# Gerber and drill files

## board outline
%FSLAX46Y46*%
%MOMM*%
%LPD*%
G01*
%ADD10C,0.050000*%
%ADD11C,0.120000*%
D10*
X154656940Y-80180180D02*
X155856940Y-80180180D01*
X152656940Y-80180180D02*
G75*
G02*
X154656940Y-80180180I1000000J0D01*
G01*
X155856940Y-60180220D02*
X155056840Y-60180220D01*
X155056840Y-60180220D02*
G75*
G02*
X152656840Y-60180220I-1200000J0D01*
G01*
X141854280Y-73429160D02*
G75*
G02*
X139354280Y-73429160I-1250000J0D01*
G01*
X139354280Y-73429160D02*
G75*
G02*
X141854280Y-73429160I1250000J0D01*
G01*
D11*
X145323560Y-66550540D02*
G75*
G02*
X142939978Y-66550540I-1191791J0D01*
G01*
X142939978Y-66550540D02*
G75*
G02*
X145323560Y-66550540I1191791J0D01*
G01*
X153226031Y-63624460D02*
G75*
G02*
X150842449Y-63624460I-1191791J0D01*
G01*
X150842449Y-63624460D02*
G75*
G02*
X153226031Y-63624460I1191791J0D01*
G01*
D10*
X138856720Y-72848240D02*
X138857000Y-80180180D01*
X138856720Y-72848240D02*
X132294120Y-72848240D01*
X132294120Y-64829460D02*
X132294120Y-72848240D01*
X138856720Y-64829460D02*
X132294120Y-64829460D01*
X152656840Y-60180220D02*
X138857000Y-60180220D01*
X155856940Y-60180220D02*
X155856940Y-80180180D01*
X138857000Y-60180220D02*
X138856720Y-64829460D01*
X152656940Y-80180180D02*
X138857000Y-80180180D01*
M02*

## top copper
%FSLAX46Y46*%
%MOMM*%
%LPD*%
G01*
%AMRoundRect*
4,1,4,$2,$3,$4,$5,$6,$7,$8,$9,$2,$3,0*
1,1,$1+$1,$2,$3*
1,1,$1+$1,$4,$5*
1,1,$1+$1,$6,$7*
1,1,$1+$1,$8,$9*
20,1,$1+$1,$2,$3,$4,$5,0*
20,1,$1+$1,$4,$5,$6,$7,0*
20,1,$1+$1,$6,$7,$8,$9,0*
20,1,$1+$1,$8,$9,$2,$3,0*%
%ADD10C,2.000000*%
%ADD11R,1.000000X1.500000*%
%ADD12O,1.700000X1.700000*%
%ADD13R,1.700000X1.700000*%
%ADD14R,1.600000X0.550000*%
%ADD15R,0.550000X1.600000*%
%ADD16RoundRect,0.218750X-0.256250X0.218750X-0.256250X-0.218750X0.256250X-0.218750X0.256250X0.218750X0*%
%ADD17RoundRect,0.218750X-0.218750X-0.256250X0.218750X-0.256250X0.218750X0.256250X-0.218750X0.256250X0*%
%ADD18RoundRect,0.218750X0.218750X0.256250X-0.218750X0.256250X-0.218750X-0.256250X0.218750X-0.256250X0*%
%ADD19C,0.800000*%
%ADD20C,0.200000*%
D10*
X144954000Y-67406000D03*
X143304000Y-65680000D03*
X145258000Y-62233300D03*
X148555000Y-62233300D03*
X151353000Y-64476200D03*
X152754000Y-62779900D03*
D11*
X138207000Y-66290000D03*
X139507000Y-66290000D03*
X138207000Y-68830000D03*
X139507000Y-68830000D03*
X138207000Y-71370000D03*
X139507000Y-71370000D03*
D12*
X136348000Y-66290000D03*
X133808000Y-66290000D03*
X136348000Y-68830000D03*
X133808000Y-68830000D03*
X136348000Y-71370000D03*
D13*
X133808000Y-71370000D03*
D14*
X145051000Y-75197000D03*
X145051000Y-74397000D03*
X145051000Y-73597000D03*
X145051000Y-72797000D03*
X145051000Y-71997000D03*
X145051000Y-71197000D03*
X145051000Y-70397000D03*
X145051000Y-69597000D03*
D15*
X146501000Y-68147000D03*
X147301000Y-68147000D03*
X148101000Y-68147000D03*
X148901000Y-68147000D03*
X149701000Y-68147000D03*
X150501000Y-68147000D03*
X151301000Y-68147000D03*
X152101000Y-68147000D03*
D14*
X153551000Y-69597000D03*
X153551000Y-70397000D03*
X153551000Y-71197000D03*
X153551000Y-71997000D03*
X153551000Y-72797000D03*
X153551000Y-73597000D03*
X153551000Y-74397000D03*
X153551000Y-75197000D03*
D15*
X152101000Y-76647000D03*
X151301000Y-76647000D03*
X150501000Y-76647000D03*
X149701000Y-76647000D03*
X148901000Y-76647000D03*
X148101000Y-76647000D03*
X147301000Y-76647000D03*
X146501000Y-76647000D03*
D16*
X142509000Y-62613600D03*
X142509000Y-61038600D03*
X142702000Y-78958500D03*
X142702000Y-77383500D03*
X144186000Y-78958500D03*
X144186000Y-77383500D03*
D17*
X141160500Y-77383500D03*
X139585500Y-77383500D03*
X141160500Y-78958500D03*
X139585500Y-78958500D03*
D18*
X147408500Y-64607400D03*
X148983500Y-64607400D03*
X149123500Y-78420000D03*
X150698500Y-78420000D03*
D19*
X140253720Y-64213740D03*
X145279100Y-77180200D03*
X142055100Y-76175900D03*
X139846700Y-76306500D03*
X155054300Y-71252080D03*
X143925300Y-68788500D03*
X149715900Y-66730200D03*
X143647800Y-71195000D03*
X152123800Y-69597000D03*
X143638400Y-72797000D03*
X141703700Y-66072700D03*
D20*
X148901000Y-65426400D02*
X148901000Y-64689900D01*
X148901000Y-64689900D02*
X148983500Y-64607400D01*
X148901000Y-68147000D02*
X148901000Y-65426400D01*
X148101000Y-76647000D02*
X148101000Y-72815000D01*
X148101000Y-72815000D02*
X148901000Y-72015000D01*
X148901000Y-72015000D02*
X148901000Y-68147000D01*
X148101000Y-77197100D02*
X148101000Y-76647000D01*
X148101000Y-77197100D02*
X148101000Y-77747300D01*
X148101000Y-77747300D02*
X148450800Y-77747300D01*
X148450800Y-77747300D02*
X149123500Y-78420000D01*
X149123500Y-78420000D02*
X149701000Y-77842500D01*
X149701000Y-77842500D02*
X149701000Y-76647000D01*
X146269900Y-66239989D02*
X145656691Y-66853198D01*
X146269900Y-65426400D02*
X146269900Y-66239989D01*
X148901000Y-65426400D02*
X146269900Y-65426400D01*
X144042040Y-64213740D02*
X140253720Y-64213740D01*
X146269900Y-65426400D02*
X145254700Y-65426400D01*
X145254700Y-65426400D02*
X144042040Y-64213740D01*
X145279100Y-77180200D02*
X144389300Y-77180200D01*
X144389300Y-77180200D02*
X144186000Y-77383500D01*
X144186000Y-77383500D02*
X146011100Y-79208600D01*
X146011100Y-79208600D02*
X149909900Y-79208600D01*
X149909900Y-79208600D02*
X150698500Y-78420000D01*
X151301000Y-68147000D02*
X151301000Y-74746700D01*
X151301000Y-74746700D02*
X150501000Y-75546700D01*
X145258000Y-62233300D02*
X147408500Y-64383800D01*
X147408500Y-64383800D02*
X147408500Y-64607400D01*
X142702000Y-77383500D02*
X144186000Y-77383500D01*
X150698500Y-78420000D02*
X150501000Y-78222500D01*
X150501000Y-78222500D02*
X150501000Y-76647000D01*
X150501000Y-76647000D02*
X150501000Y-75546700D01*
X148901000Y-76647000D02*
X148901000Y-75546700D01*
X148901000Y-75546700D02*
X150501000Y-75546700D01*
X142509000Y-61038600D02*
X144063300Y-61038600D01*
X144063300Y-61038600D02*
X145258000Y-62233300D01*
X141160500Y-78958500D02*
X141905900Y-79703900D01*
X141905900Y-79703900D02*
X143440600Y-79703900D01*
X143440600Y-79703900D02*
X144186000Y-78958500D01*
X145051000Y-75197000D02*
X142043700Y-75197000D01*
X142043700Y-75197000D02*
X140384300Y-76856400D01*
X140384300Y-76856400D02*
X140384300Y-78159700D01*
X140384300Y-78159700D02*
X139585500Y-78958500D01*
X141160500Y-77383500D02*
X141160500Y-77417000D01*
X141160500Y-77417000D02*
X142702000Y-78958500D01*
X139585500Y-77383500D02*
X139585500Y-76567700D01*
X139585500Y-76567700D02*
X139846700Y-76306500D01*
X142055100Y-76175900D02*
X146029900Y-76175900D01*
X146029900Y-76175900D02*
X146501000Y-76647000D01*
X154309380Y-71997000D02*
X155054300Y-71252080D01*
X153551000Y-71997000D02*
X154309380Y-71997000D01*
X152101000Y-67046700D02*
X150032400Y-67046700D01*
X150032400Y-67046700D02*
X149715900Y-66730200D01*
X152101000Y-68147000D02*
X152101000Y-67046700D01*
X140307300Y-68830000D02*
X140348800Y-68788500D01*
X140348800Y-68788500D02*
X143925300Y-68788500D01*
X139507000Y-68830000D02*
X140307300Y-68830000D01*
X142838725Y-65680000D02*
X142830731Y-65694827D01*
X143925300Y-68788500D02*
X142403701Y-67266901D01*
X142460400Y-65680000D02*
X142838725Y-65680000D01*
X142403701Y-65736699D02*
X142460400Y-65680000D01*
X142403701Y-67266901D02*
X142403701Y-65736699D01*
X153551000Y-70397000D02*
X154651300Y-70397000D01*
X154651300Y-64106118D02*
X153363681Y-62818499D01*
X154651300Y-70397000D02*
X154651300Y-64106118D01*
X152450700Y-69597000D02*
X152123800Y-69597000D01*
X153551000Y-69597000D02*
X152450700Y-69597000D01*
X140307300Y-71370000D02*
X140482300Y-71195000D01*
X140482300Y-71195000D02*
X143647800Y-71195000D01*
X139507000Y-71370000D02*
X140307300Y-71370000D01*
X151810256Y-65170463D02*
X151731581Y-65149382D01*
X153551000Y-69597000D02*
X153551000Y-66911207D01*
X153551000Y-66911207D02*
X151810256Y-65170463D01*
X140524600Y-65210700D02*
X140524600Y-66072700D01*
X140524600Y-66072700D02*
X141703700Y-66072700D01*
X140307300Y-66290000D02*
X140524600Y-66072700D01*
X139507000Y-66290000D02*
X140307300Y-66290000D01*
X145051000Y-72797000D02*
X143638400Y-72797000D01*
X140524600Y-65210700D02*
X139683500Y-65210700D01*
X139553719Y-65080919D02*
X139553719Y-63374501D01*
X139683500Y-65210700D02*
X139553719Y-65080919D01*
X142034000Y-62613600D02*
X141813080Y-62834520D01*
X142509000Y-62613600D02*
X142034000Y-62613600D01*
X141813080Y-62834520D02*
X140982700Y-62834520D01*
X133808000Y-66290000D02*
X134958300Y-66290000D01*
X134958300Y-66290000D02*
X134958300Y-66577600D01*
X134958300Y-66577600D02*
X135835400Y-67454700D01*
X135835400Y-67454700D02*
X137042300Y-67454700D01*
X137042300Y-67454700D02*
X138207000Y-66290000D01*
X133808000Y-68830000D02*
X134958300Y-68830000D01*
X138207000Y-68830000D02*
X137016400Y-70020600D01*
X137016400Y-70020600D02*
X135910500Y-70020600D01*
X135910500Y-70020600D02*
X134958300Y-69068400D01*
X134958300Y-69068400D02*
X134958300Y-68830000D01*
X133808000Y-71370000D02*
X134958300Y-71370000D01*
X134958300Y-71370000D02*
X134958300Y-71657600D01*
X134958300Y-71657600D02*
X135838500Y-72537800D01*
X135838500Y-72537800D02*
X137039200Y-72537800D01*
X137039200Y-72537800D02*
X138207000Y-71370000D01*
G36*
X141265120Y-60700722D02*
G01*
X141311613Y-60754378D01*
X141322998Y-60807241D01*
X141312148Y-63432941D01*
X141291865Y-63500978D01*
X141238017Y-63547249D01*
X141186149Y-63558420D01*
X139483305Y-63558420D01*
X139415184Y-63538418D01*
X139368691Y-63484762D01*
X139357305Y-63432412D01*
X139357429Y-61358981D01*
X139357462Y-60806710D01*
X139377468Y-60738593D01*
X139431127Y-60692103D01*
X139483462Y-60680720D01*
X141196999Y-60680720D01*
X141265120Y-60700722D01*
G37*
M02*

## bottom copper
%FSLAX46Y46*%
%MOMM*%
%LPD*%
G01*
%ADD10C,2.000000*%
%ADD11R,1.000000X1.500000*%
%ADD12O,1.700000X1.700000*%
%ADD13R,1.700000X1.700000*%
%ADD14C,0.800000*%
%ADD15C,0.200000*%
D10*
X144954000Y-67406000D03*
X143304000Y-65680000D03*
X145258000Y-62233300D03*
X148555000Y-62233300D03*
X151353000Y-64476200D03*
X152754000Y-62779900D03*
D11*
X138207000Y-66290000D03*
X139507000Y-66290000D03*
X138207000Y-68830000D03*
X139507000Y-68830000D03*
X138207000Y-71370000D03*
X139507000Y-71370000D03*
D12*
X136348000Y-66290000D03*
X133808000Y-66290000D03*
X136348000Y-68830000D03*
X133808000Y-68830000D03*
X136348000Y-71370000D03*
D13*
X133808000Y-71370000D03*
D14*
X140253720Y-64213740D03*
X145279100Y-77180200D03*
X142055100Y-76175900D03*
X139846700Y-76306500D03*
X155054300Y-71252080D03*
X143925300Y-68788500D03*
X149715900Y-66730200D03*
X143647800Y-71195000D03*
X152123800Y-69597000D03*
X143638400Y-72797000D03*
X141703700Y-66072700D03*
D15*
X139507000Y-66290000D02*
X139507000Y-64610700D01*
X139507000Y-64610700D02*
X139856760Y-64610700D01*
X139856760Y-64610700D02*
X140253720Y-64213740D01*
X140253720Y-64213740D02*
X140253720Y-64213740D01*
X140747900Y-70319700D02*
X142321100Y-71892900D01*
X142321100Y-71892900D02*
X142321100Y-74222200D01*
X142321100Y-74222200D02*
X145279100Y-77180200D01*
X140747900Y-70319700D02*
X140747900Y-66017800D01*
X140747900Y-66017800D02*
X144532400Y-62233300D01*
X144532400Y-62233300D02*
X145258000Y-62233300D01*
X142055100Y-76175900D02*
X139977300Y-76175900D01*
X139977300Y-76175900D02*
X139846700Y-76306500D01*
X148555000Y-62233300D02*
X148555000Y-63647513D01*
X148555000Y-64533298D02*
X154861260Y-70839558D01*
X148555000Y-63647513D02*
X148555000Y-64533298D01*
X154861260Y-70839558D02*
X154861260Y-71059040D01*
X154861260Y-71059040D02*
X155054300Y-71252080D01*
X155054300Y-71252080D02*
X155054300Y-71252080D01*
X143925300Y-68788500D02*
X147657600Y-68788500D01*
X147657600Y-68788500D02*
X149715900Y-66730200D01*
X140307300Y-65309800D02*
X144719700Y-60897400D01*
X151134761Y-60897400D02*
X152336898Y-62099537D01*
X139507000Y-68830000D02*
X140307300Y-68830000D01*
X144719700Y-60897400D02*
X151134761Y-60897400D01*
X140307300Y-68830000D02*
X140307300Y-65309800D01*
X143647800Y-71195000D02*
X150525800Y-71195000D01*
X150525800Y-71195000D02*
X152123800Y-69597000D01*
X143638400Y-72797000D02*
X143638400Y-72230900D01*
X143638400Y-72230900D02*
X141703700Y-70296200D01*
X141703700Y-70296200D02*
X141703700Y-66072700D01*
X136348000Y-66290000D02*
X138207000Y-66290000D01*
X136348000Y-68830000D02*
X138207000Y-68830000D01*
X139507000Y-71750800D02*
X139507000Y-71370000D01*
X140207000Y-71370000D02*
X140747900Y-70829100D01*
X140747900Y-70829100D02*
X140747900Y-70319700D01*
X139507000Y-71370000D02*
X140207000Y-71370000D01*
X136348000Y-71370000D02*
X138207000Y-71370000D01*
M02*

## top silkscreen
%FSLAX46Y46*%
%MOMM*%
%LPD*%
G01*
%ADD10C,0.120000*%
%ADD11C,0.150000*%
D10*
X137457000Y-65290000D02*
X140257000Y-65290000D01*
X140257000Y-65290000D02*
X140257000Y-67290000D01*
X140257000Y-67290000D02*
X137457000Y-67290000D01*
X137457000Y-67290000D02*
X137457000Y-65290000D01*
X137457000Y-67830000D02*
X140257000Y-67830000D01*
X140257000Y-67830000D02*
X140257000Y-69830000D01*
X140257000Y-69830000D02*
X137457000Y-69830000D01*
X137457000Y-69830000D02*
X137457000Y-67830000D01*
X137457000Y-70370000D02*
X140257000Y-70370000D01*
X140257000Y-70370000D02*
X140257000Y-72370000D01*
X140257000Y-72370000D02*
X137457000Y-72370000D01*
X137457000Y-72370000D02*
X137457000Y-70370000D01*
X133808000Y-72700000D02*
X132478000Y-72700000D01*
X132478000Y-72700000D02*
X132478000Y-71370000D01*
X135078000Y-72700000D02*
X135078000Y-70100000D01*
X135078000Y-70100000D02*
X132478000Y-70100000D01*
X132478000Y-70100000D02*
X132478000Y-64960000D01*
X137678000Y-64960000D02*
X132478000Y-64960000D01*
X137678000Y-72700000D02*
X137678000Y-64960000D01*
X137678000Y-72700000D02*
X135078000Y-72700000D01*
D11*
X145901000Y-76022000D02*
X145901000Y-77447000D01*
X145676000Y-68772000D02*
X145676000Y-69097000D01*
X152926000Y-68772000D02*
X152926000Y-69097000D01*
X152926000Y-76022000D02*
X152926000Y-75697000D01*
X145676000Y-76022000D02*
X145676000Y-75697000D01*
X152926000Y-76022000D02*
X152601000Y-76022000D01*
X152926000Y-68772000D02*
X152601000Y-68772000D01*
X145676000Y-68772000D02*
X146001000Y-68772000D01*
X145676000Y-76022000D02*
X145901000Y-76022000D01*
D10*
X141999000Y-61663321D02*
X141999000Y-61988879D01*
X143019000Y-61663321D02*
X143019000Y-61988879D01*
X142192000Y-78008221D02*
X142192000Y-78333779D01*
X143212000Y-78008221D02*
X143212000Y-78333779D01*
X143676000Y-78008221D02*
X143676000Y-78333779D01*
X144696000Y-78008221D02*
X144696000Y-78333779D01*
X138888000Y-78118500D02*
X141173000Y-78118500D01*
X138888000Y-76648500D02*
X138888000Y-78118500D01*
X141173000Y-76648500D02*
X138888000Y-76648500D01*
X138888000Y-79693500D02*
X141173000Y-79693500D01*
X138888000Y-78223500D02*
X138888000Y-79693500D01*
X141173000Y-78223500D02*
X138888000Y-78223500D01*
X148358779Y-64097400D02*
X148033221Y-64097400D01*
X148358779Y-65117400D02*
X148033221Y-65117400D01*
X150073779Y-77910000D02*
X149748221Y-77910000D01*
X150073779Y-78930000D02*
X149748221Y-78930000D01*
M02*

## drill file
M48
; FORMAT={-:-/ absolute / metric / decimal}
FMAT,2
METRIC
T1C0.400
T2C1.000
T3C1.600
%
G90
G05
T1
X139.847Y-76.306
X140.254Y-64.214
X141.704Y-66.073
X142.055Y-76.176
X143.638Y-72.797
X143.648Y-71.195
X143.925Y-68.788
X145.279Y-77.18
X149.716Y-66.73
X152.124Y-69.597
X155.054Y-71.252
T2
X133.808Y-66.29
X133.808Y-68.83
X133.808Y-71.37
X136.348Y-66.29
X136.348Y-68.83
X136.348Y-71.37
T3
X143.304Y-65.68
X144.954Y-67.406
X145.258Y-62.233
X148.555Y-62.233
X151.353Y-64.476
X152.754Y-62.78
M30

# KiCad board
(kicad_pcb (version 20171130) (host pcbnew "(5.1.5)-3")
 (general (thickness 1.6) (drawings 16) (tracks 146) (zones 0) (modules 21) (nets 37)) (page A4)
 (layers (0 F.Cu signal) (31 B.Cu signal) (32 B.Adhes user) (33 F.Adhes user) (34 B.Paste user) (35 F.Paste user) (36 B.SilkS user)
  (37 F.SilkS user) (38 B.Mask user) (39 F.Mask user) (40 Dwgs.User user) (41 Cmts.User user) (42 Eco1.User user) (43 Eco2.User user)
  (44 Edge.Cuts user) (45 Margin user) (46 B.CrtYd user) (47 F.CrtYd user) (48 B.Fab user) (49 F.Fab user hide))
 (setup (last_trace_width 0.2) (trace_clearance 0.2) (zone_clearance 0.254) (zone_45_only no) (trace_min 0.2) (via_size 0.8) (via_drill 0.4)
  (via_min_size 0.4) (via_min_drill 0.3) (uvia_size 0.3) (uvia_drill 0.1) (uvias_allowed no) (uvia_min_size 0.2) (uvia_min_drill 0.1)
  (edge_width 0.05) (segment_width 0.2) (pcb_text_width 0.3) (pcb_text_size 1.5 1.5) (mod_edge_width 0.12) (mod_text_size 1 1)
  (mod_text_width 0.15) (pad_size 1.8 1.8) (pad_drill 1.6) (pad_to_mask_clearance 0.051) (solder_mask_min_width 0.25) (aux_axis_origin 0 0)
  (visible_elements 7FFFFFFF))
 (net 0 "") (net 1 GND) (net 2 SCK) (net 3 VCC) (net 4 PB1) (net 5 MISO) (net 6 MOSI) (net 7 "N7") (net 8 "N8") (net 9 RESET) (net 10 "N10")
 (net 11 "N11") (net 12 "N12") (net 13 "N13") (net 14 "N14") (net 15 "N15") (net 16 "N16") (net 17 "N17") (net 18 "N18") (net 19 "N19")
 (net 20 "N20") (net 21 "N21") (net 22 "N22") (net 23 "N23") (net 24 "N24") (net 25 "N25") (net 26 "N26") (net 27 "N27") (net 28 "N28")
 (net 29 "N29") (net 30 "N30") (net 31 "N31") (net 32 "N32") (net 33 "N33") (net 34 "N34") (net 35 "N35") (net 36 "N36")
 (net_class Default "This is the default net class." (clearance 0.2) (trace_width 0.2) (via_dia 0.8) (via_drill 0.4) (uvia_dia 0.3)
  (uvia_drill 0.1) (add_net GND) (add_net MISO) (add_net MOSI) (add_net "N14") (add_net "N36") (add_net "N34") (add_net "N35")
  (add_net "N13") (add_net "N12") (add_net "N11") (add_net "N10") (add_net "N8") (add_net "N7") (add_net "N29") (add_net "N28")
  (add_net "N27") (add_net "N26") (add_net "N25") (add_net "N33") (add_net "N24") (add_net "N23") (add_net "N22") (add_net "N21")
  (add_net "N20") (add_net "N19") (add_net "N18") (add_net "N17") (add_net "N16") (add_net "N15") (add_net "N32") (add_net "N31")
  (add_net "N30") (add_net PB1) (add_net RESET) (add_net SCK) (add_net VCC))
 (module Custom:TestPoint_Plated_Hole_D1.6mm (layer F.Cu) (at 144.954 67.406 180)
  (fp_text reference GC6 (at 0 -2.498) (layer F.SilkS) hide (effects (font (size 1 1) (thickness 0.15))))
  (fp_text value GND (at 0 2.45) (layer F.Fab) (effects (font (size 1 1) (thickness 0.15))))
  (pad 1 thru_hole circle (at 0 0 180) (size 2 2) (drill 1.6) (layers *.Cu *.Mask) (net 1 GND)))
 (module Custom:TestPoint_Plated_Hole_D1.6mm (layer F.Cu) (at 143.304 65.68 180)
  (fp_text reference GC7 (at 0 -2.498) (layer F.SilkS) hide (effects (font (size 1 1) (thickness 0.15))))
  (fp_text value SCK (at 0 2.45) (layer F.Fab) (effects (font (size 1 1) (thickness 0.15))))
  (pad 1 thru_hole circle (at 0 0 180) (size 2 2) (drill 1.6) (layers *.Cu *.Mask) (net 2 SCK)))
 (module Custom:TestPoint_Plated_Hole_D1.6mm (layer F.Cu) (at 145.258 62.2333 180)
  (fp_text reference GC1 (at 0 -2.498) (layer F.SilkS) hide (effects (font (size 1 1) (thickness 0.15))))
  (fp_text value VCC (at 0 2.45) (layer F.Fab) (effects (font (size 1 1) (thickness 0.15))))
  (pad 1 thru_hole circle (at 0 0 180) (size 2 2) (drill 1.6) (layers *.Cu *.Mask) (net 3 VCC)))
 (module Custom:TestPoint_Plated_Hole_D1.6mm (layer F.Cu) (at 148.555 62.2333 180)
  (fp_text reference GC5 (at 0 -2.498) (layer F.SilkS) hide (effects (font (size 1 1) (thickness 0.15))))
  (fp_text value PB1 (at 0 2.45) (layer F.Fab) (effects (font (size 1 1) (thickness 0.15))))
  (pad 1 thru_hole circle (at 0 0 180) (size 2 2) (drill 1.6) (layers *.Cu *.Mask) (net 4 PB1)))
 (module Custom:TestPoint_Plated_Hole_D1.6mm (layer F.Cu) (at 151.353 64.4762 180)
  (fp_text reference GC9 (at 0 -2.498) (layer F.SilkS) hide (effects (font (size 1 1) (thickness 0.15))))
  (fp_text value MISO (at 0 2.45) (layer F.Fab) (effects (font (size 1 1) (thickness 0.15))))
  (pad 1 thru_hole circle (at 0 0 180) (size 2 2) (drill 1.6) (layers *.Cu *.Mask) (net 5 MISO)))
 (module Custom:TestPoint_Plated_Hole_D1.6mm (layer F.Cu) (at 152.754 62.7799 180)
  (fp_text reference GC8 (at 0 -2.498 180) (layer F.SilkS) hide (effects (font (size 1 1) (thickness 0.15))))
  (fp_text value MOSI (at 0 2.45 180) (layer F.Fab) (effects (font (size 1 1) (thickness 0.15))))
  (pad 1 thru_hole circle (at 0 0 180) (size 2 2) (drill 1.6) (layers *.Cu *.Mask) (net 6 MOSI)))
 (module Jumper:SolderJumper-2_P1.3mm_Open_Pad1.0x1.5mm (layer B.Cu) (at 138.857 66.29)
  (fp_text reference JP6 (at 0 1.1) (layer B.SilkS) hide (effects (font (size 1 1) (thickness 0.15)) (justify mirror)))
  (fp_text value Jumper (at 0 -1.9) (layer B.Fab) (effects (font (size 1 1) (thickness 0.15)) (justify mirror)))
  (pad 1 smd rect (at -0.65 0) (size 1 1.5) (layers B.Cu B.Mask) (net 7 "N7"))
  (pad 2 smd rect (at 0.65 0) (size 1 1.5) (layers B.Cu B.Mask) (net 1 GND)))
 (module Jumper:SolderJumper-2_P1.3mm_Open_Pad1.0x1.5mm (layer F.Cu) (at 138.857 66.29)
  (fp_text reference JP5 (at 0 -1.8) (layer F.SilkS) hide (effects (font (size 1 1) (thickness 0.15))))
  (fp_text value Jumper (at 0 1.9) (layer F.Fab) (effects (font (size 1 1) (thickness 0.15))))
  (fp_line (start -1.4 -1) (end 1.4 -1) (layer F.SilkS) (width 0.12))
  (fp_line (start 1.4 -1) (end 1.4 1) (layer F.SilkS) (width 0.12))
  (fp_line (start 1.4 1) (end -1.4 1) (layer F.SilkS) (width 0.12))
  (fp_line (start -1.4 1) (end -1.4 -1) (layer F.SilkS) (width 0.12))
  (pad 1 smd rect (at -0.65 0) (size 1 1.5) (layers F.Cu F.Mask) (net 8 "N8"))
  (pad 2 smd rect (at 0.65 0) (size 1 1.5) (layers F.Cu F.Mask) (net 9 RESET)))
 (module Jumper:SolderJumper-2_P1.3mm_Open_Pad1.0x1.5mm (layer B.Cu) (at 138.857 68.83)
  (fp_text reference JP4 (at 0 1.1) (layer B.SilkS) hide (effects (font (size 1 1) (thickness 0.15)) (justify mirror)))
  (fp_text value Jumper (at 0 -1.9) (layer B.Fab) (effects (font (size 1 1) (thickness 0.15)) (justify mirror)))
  (pad 1 smd rect (at -0.65 0) (size 1 1.5) (layers B.Cu B.Mask) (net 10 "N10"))
  (pad 2 smd rect (at 0.65 0) (size 1 1.5) (layers B.Cu B.Mask) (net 6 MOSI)))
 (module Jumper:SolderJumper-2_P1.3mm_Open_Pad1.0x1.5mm (layer F.Cu) (at 138.857 68.83)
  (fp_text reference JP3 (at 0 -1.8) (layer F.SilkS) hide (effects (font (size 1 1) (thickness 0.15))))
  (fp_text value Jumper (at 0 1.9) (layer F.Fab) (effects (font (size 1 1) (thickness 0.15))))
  (fp_line (start -1.4 -1) (end 1.4 -1) (layer F.SilkS) (width 0.12))
  (fp_line (start 1.4 -1) (end 1.4 1) (layer F.SilkS) (width 0.12))
  (fp_line (start 1.4 1) (end -1.4 1) (layer F.SilkS) (width 0.12))
  (fp_line (start -1.4 1) (end -1.4 -1) (layer F.SilkS) (width 0.12))
  (pad 1 smd rect (at -0.65 0) (size 1 1.5) (layers F.Cu F.Mask) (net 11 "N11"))
  (pad 2 smd rect (at 0.65 0) (size 1 1.5) (layers F.Cu F.Mask) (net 2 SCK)))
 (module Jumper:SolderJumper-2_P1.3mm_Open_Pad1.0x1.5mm (layer B.Cu) (at 138.857 71.37)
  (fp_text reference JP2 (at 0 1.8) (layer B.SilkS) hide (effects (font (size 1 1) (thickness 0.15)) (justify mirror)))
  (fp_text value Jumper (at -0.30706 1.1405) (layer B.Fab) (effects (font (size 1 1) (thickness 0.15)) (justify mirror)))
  (pad 1 smd rect (at -0.65 0) (size 1 1.5) (layers B.Cu B.Mask) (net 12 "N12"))
  (pad 2 smd rect (at 0.65 0) (size 1 1.5) (layers B.Cu B.Mask) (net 3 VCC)))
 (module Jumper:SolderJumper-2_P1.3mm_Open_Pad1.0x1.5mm (layer F.Cu) (at 138.857 71.37)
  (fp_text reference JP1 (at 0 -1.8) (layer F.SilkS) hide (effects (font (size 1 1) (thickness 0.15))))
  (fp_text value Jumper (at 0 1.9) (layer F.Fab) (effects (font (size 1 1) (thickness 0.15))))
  (fp_line (start -1.4 -1) (end 1.4 -1) (layer F.SilkS) (width 0.12))
  (fp_line (start 1.4 -1) (end 1.4 1) (layer F.SilkS) (width 0.12))
  (fp_line (start 1.4 1) (end -1.4 1) (layer F.SilkS) (width 0.12))
  (fp_line (start -1.4 1) (end -1.4 -1) (layer F.SilkS) (width 0.12))
  (pad 1 smd rect (at -0.65 0) (size 1 1.5) (layers F.Cu F.Mask) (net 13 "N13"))
  (pad 2 smd rect (at 0.65 0) (size 1 1.5) (layers F.Cu F.Mask) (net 5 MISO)))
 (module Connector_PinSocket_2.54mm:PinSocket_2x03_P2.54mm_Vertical (layer F.Cu) (at 133.808 71.37 180)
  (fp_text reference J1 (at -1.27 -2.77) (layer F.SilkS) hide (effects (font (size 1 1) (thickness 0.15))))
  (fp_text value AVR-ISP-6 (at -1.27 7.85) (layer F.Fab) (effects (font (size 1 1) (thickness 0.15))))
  (fp_line (start 0 -1.33) (end 1.33 -1.33) (layer F.SilkS) (width 0.12))
  (fp_line (start 1.33 -1.33) (end 1.33 0) (layer F.SilkS) (width 0.12))
  (fp_line (start -1.27 -1.33) (end -1.27 1.27) (layer F.SilkS) (width 0.12))
  (fp_line (start -1.27 1.27) (end 1.33 1.27) (layer F.SilkS) (width 0.12))
  (fp_line (start 1.33 1.27) (end 1.33 6.41) (layer F.SilkS) (width 0.12))
  (fp_line (start -3.87 6.41) (end 1.33 6.41) (layer F.SilkS) (width 0.12))
  (fp_line (start -3.87 -1.33) (end -3.87 6.41) (layer F.SilkS) (width 0.12))
  (fp_line (start -3.87 -1.33) (end -1.27 -1.33) (layer F.SilkS) (width 0.12))
  (pad 6 thru_hole oval (at -2.54 5.08 180) (size 1.7 1.7) (drill 1) (layers *.Cu *.Mask) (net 7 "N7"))
  (pad 5 thru_hole oval (at 0 5.08 180) (size 1.7 1.7) (drill 1) (layers *.Cu *.Mask) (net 8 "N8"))
  (pad 4 thru_hole oval (at -2.54 2.54 180) (size 1.7 1.7) (drill 1) (layers *.Cu *.Mask) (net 10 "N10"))
  (pad 3 thru_hole oval (at 0 2.54 180) (size 1.7 1.7) (drill 1) (layers *.Cu *.Mask) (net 11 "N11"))
  (pad 2 thru_hole oval (at -2.54 0 180) (size 1.7 1.7) (drill 1) (layers *.Cu *.Mask) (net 12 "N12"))
  (pad 1 thru_hole rect (at 0 0 180) (size 1.7 1.7) (drill 1) (layers *.Cu *.Mask) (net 13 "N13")))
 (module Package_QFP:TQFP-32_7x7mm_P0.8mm (layer F.Cu) (at 149.301 72.397 90)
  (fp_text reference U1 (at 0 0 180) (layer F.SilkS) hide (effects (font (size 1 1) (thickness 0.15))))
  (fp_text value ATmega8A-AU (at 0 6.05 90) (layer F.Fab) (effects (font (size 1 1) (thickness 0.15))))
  (fp_line (start -3.625 -3.4) (end -5.05 -3.4) (layer F.SilkS) (width 0.15))
  (fp_line (start 3.625 -3.625) (end 3.3 -3.625) (layer F.SilkS) (width 0.15))
  (fp_line (start 3.625 3.625) (end 3.3 3.625) (layer F.SilkS) (width 0.15))
  (fp_line (start -3.625 3.625) (end -3.3 3.625) (layer F.SilkS) (width 0.15))
  (fp_line (start -3.625 -3.625) (end -3.3 -3.625) (layer F.SilkS) (width 0.15))
  (fp_line (start -3.625 3.625) (end -3.625 3.3) (layer F.SilkS) (width 0.15))
  (fp_line (start 3.625 3.625) (end 3.625 3.3) (layer F.SilkS) (width 0.15))
  (fp_line (start 3.625 -3.625) (end 3.625 -3.3) (layer F.SilkS) (width 0.15))
  (fp_line (start -3.625 -3.625) (end -3.625 -3.4) (layer F.SilkS) (width 0.15))
  (pad 32 smd rect (at -2.8 -4.25 180) (size 1.6 0.55) (layers F.Cu F.Paste F.Mask) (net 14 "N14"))
  (pad 31 smd rect (at -2 -4.25 180) (size 1.6 0.55) (layers F.Cu F.Paste F.Mask) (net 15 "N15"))
  (pad 30 smd rect (at -1.2 -4.25 180) (size 1.6 0.55) (layers F.Cu F.Paste F.Mask) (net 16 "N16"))
  (pad 29 smd rect (at -0.4 -4.25 180) (size 1.6 0.55) (layers F.Cu F.Paste F.Mask) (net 9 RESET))
  (pad 28 smd rect (at 0.4 -4.25 180) (size 1.6 0.55) (layers F.Cu F.Paste F.Mask) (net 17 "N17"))
  (pad 27 smd rect (at 1.2 -4.25 180) (size 1.6 0.55) (layers F.Cu F.Paste F.Mask) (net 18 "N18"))
  (pad 26 smd rect (at 2 -4.25 180) (size 1.6 0.55) (layers F.Cu F.Paste F.Mask) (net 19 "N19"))
  (pad 25 smd rect (at 2.8 -4.25 180) (size 1.6 0.55) (layers F.Cu F.Paste F.Mask) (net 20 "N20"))
  (pad 24 smd rect (at 4.25 -2.8 90) (size 1.6 0.55) (layers F.Cu F.Paste F.Mask) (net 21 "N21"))
  (pad 23 smd rect (at 4.25 -2 90) (size 1.6 0.55) (layers F.Cu F.Paste F.Mask) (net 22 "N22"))
  (pad 22 smd rect (at 4.25 -1.2 90) (size 1.6 0.55) (layers F.Cu F.Paste F.Mask) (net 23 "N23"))
  (pad 21 smd rect (at 4.25 -0.4 90) (size 1.6 0.55) (layers F.Cu F.Paste F.Mask) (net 1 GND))
  (pad 20 smd rect (at 4.25 0.4 90) (size 1.6 0.55) (layers F.Cu F.Paste F.Mask) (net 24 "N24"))
  (pad 19 smd rect (at 4.25 1.2 90) (size 1.6 0.55) (layers F.Cu F.Paste F.Mask) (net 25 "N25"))
  (pad 18 smd rect (at 4.25 2 90) (size 1.6 0.55) (layers F.Cu F.Paste F.Mask) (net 3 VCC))
  (pad 17 smd rect (at 4.25 2.8 90) (size 1.6 0.55) (layers F.Cu F.Paste F.Mask) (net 2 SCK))
  (pad 16 smd rect (at 2.8 4.25 180) (size 1.6 0.55) (layers F.Cu F.Paste F.Mask) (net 5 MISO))
  (pad 15 smd rect (at 2 4.25 180) (size 1.6 0.55) (layers F.Cu F.Paste F.Mask) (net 6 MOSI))
  (pad 14 smd rect (at 1.2 4.25 180) (size 1.6 0.55) (layers F.Cu F.Paste F.Mask) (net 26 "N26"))
  (pad 13 smd rect (at 0.4 4.25 180) (size 1.6 0.55) (layers F.Cu F.Paste F.Mask) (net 4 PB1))
  (pad 12 smd rect (at -0.4 4.25 180) (size 1.6 0.55) (layers F.Cu F.Paste F.Mask) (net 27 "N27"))
  (pad 11 smd rect (at -1.2 4.25 180) (size 1.6 0.55) (layers F.Cu F.Paste F.Mask) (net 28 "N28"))
  (pad 10 smd rect (at -2 4.25 180) (size 1.6 0.55) (layers F.Cu F.Paste F.Mask) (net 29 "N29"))
  (pad 9 smd rect (at -2.8 4.25 180) (size 1.6 0.55) (layers F.Cu F.Paste F.Mask) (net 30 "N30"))
  (pad 8 smd rect (at -4.25 2.8 90) (size 1.6 0.55) (layers F.Cu F.Paste F.Mask) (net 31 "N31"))
  (pad 7 smd rect (at -4.25 2 90) (size 1.6 0.55) (layers F.Cu F.Paste F.Mask) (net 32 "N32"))
  (pad 6 smd rect (at -4.25 1.2 90) (size 1.6 0.55) (layers F.Cu F.Paste F.Mask) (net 3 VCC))
  (pad 5 smd rect (at -4.25 0.4 90) (size 1.6 0.55) (layers F.Cu F.Paste F.Mask) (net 1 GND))
  (pad 4 smd rect (at -4.25 -0.4 90) (size 1.6 0.55) (layers F.Cu F.Paste F.Mask) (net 3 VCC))
  (pad 3 smd rect (at -4.25 -1.2 90) (size 1.6 0.55) (layers F.Cu F.Paste F.Mask) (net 1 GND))
  (pad 2 smd rect (at -4.25 -2 90) (size 1.6 0.55) (layers F.Cu F.Paste F.Mask) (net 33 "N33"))
  (pad 1 smd rect (at -4.25 -2.8 90) (size 1.6 0.55) (layers F.Cu F.Paste F.Mask) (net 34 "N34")))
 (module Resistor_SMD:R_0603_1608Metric (layer F.Cu) (at 142.509 61.8261 270)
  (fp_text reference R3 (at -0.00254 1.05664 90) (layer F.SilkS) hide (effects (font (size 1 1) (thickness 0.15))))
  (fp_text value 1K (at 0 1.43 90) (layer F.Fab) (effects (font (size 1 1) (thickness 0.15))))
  (fp_line (start -0.162779 0.51) (end 0.162779 0.51) (layer F.SilkS) (width 0.12))
  (fp_line (start -0.162779 -0.51) (end 0.162779 -0.51) (layer F.SilkS) (width 0.12))
  (pad 2 smd roundrect (at 0.7875 0 270) (size 0.875 0.95) (layers F.Cu F.Paste F.Mask) (roundrect_rratio 0.25) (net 9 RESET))
  (pad 1 smd roundrect (at -0.7875 0 270) (size 0.875 0.95) (layers F.Cu F.Paste F.Mask) (roundrect_rratio 0.25) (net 3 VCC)))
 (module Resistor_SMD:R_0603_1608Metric (layer F.Cu) (at 142.702 78.171 270)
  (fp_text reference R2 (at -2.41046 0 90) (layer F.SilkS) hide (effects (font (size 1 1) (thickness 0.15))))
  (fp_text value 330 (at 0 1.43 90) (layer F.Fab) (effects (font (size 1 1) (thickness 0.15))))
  (fp_line (start -0.162779 0.51) (end 0.162779 0.51) (layer F.SilkS) (width 0.12))
  (fp_line (start -0.162779 -0.51) (end 0.162779 -0.51) (layer F.SilkS) (width 0.12))
  (pad 2 smd roundrect (at 0.7875 0 270) (size 0.875 0.95) (layers F.Cu F.Paste F.Mask) (roundrect_rratio 0.25) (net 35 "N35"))
  (pad 1 smd roundrect (at -0.7875 0 270) (size 0.875 0.95) (layers F.Cu F.Paste F.Mask) (roundrect_rratio 0.25) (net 3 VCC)))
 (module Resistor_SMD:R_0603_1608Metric (layer F.Cu) (at 144.186 78.171 270)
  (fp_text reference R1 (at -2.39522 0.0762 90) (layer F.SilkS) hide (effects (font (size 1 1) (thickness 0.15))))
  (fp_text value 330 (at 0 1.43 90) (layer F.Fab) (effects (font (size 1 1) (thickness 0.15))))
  (fp_line (start -0.162779 0.51) (end 0.162779 0.51) (layer F.SilkS) (width 0.12))
  (fp_line (start -0.162779 -0.51) (end 0.162779 -0.51) (layer F.SilkS) (width 0.12))
  (pad 2 smd roundrect (at 0.7875 0 270) (size 0.875 0.95) (layers F.Cu F.Paste F.Mask) (roundrect_rratio 0.25) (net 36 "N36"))
  (pad 1 smd roundrect (at -0.7875 0 270) (size 0.875 0.95) (layers F.Cu F.Paste F.Mask) (roundrect_rratio 0.25) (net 3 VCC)))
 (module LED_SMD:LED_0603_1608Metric (layer F.Cu) (at 140.373 77.3835)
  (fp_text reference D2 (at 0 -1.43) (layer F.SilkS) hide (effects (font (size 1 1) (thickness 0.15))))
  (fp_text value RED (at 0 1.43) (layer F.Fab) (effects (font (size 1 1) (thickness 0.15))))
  (fp_line (start -1.485 0.735) (end 0.8 0.735) (layer F.SilkS) (width 0.12))
  (fp_line (start -1.485 -0.735) (end -1.485 0.735) (layer F.SilkS) (width 0.12))
  (fp_line (start 0.8 -0.735) (end -1.485 -0.735) (layer F.SilkS) (width 0.12))
  (pad 2 smd roundrect (at 0.7875 0) (size 0.875 0.95) (layers F.Cu F.Paste F.Mask) (roundrect_rratio 0.25) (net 35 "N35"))
  (pad 1 smd roundrect (at -0.7875 0) (size 0.875 0.95) (layers F.Cu F.Paste F.Mask) (roundrect_rratio 0.25) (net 34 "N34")))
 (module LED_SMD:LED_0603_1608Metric (layer F.Cu) (at 140.373 78.9585)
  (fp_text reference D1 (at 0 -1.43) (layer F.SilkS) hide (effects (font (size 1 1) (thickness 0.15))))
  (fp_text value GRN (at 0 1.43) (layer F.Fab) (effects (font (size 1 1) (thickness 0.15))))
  (fp_line (start -1.485 0.735) (end 0.8 0.735) (layer F.SilkS) (width 0.12))
  (fp_line (start -1.485 -0.735) (end -1.485 0.735) (layer F.SilkS) (width 0.12))
  (fp_line (start 0.8 -0.735) (end -1.485 -0.735) (layer F.SilkS) (width 0.12))
  (pad 2 smd roundrect (at 0.7875 0) (size 0.875 0.95) (layers F.Cu F.Paste F.Mask) (roundrect_rratio 0.25) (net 36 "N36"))
  (pad 1 smd roundrect (at -0.7875 0) (size 0.875 0.95) (layers F.Cu F.Paste F.Mask) (roundrect_rratio 0.25) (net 14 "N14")))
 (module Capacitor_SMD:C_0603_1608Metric (layer F.Cu) (at 148.196 64.6074 180)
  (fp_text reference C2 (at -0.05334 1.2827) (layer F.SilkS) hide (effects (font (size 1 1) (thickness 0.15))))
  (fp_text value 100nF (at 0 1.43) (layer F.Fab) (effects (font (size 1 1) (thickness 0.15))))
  (fp_line (start -0.162779 0.51) (end 0.162779 0.51) (layer F.SilkS) (width 0.12))
  (fp_line (start -0.162779 -0.51) (end 0.162779 -0.51) (layer F.SilkS) (width 0.12))
  (pad 2 smd roundrect (at 0.7875 0 180) (size 0.875 0.95) (layers F.Cu F.Paste F.Mask) (roundrect_rratio 0.25) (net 3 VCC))
  (pad 1 smd roundrect (at -0.7875 0 180) (size 0.875 0.95) (layers F.Cu F.Paste F.Mask) (roundrect_rratio 0.25) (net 1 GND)))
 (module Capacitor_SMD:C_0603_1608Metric (layer F.Cu) (at 149.911 78.42 180)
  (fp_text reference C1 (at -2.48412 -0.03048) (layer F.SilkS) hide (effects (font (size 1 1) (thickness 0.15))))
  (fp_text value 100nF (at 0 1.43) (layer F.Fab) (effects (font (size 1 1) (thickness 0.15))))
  (fp_line (start -0.162779 0.51) (end 0.162779 0.51) (layer F.SilkS) (width 0.12))
  (fp_line (start -0.162779 -0.51) (end 0.162779 -0.51) (layer F.SilkS) (width 0.12))
  (pad 2 smd roundrect (at 0.7875 0 180) (size 0.875 0.95) (layers F.Cu F.Paste F.Mask) (roundrect_rratio 0.25) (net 1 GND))
  (pad 1 smd roundrect (at -0.7875 0 180) (size 0.875 0.95) (layers F.Cu F.Paste F.Mask) (roundrect_rratio 0.25) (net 3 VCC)))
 (gr_line (start 154.65694 80.18018) (end 155.85694 80.18018) (layer Edge.Cuts) (width 0.05))
 (gr_arc (start 153.65694 80.18018) (end 154.65694 80.18018) (angle -180) (layer Edge.Cuts) (width 0.05))
 (gr_line (start 155.85694 60.18022) (end 155.05684 60.18022) (layer Edge.Cuts) (width 0.05))
 (gr_arc (start 153.85684 60.18022) (end 152.65684 60.18022) (angle -180) (layer Edge.Cuts) (width 0.05))
 (gr_circle (center 140.60428 73.42916) (end 140.60428 74.67916) (layer Edge.Cuts) (width 0.05))
 (gr_circle (center 144.131769 66.55054) (end 145.32356 66.55054) (layer Edge.Cuts) (width 0.12))
 (gr_circle (center 152.03424 63.62446) (end 153.226031 63.62446) (layer Edge.Cuts) (width 0.12))
 (gr_line (start 138.85672 72.84824) (end 138.857 80.18018) (layer Edge.Cuts) (width 0.05))
 (gr_line (start 138.85672 72.84824) (end 132.29412 72.84824) (layer Edge.Cuts) (width 0.05))
 (gr_line (start 132.29412 64.82946) (end 132.29412 72.84824) (layer Edge.Cuts) (width 0.05))
 (gr_line (start 138.85672 64.82946) (end 132.29412 64.82946) (layer Edge.Cuts) (width 0.05))
 (gr_line (start 152.65684 60.18022) (end 138.857 60.18022) (layer Edge.Cuts) (width 0.05))
 (gr_line (start 155.85694 60.18022) (end 155.85694 80.18018) (layer Edge.Cuts) (width 0.05))
 (gr_line (start 138.857 60.18022) (end 138.85672 64.82946) (layer Edge.Cuts) (width 0.05))
 (gr_line (start 152.65694 80.18018) (end 138.857 80.18018) (layer Edge.Cuts) (width 0.05))
 (segment (start 139.507 66.29) (end 139.507 64.6107) (width 0.2) (layer B.Cu) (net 1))
 (segment (start 148.901 65.4264) (end 148.901 64.6899) (width 0.2) (layer F.Cu) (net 1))
 (segment (start 148.901 64.6899) (end 148.9835 64.6074) (width 0.2) (layer F.Cu) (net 1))
 (segment (start 148.901 68.147) (end 148.901 65.4264) (width 0.2) (layer F.Cu) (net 1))
 (segment (start 148.101 76.647) (end 148.101 72.815) (width 0.2) (layer F.Cu) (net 1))
 (segment (start 148.101 72.815) (end 148.901 72.015) (width 0.2) (layer F.Cu) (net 1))
 (segment (start 148.901 72.015) (end 148.901 68.147) (width 0.2) (layer F.Cu) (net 1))
 (segment (start 148.101 77.1971) (end 148.101 76.647) (width 0.2) (layer F.Cu) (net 1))
 (segment (start 148.101 77.1971) (end 148.101 77.7473) (width 0.2) (layer F.Cu) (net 1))
 (segment (start 148.101 77.7473) (end 148.4508 77.7473) (width 0.2) (layer F.Cu) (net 1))
 (segment (start 148.4508 77.7473) (end 149.1235 78.42) (width 0.2) (layer F.Cu) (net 1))
 (segment (start 149.1235 78.42) (end 149.701 77.8425) (width 0.2) (layer F.Cu) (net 1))
 (segment (start 149.701 77.8425) (end 149.701 76.647) (width 0.2) (layer F.Cu) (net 1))
 (segment (start 146.2699 66.239989) (end 145.656691 66.853198) (width 0.2) (layer F.Cu) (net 1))
 (segment (start 146.2699 65.4264) (end 146.2699 66.239989) (width 0.2) (layer F.Cu) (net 1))
 (segment (start 148.901 65.4264) (end 146.2699 65.4264) (width 0.2) (layer F.Cu) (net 1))
 (segment (start 139.507 64.6107) (end 139.85676 64.6107) (width 0.2) (layer B.Cu) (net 1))
 (segment (start 139.85676 64.6107) (end 140.25372 64.21374) (width 0.2) (layer B.Cu) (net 1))
 (segment (start 140.25372 64.21374) (end 140.25372 64.21374) (width 0.2) (layer B.Cu) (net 1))
 (via (at 140.25372 64.21374) (size 0.8) (drill 0.4) (layers F.Cu B.Cu) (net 1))
 (segment (start 144.04204 64.21374) (end 140.25372 64.21374) (width 0.2) (layer F.Cu) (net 1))
 (segment (start 146.2699 65.4264) (end 145.2547 65.4264) (width 0.2) (layer F.Cu) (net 1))
 (segment (start 145.2547 65.4264) (end 144.04204 64.21374) (width 0.2) (layer F.Cu) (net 1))
 (segment (start 145.2791 77.1802) (end 144.3893 77.1802) (width 0.2) (layer F.Cu) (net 3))
 (segment (start 144.3893 77.1802) (end 144.186 77.3835) (width 0.2) (layer F.Cu) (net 3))
 (segment (start 140.7479 70.3197) (end 142.3211 71.8929) (width 0.2) (layer B.Cu) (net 3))
 (segment (start 142.3211 71.8929) (end 142.3211 74.2222) (width 0.2) (layer B.Cu) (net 3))
 (segment (start 142.3211 74.2222) (end 145.2791 77.1802) (width 0.2) (layer B.Cu) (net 3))
 (segment (start 140.7479 70.3197) (end 140.7479 66.0178) (width 0.2) (layer B.Cu) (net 3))
 (segment (start 140.7479 66.0178) (end 144.5324 62.2333) (width 0.2) (layer B.Cu) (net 3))
 (segment (start 144.5324 62.2333) (end 145.258 62.2333) (width 0.2) (layer B.Cu) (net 3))
 (segment (start 144.186 77.3835) (end 146.0111 79.2086) (width 0.2) (layer F.Cu) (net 3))
 (segment (start 146.0111 79.2086) (end 149.9099 79.2086) (width 0.2) (layer F.Cu) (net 3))
 (segment (start 149.9099 79.2086) (end 150.6985 78.42) (width 0.2) (layer F.Cu) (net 3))
 (segment (start 151.301 68.147) (end 151.301 74.7467) (width 0.2) (layer F.Cu) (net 3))
 (segment (start 151.301 74.7467) (end 150.501 75.5467) (width 0.2) (layer F.Cu) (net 3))
 (segment (start 145.258 62.2333) (end 147.4085 64.3838) (width 0.2) (layer F.Cu) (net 3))
 (segment (start 147.4085 64.3838) (end 147.4085 64.6074) (width 0.2) (layer F.Cu) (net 3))
 (segment (start 142.702 77.3835) (end 144.186 77.3835) (width 0.2) (layer F.Cu) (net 3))
 (segment (start 150.6985 78.42) (end 150.501 78.2225) (width 0.2) (layer F.Cu) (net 3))
 (segment (start 150.501 78.2225) (end 150.501 76.647) (width 0.2) (layer F.Cu) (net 3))
 (segment (start 150.501 76.647) (end 150.501 75.5467) (width 0.2) (layer F.Cu) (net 3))
 (segment (start 148.901 76.647) (end 148.901 75.5467) (width 0.2) (layer F.Cu) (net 3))
 (segment (start 148.901 75.5467) (end 150.501 75.5467) (width 0.2) (layer F.Cu) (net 3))
 (segment (start 142.509 61.0386) (end 144.0633 61.0386) (width 0.2) (layer F.Cu) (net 3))
 (segment (start 144.0633 61.0386) (end 145.258 62.2333) (width 0.2) (layer F.Cu) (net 3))
 (via (at 145.2791 77.1802) (size 0.8) (layers F.Cu B.Cu) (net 3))
 (segment (start 141.1605 78.9585) (end 141.9059 79.7039) (width 0.2) (layer F.Cu) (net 36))
 (segment (start 141.9059 79.7039) (end 143.4406 79.7039) (width 0.2) (layer F.Cu) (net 36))
 (segment (start 143.4406 79.7039) (end 144.186 78.9585) (width 0.2) (layer F.Cu) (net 36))
 (segment (start 145.051 75.197) (end 142.0437 75.197) (width 0.2) (layer F.Cu) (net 14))
 (segment (start 142.0437 75.197) (end 140.3843 76.8564) (width 0.2) (layer F.Cu) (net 14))
 (segment (start 140.3843 76.8564) (end 140.3843 78.1597) (width 0.2) (layer F.Cu) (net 14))
 (segment (start 140.3843 78.1597) (end 139.5855 78.9585) (width 0.2) (layer F.Cu) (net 14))
 (segment (start 141.1605 77.3835) (end 141.1605 77.417) (width 0.2) (layer F.Cu) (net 35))
 (segment (start 141.1605 77.417) (end 142.702 78.9585) (width 0.2) (layer F.Cu) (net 35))
 (segment (start 139.5855 77.3835) (end 139.5855 76.5677) (width 0.2) (layer F.Cu) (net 34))
 (segment (start 139.5855 76.5677) (end 139.8467 76.3065) (width 0.2) (layer F.Cu) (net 34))
 (segment (start 142.0551 76.1759) (end 139.9773 76.1759) (width 0.2) (layer B.Cu) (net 34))
 (segment (start 139.9773 76.1759) (end 139.8467 76.3065) (width 0.2) (layer B.Cu) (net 34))
 (segment (start 142.0551 76.1759) (end 146.0299 76.1759) (width 0.2) (layer F.Cu) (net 34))
 (segment (start 146.0299 76.1759) (end 146.501 76.647) (width 0.2) (layer F.Cu) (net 34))
 (via (at 142.0551 76.1759) (size 0.8) (layers F.Cu B.Cu) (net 34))
 (via (at 139.8467 76.3065) (size 0.8) (layers F.Cu B.Cu) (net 34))
 (segment (start 148.555 62.2333) (end 148.555 63.647513) (width 0.2) (layer B.Cu) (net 4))
 (segment (start 148.555 64.533298) (end 154.86126 70.839558) (width 0.2) (layer B.Cu) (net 4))
 (segment (start 148.555 63.647513) (end 148.555 64.533298) (width 0.2) (layer B.Cu) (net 4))
 (segment (start 154.86126 70.839558) (end 154.86126 71.05904) (width 0.2) (layer B.Cu) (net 4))
 (segment (start 154.86126 71.05904) (end 155.0543 71.25208) (width 0.2) (layer B.Cu) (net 4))
 (segment (start 155.0543 71.25208) (end 155.0543 71.25208) (width 0.2) (layer B.Cu) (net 4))
 (via (at 155.0543 71.25208) (size 0.8) (drill 0.4) (layers F.Cu B.Cu) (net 4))
 (segment (start 154.30938 71.997) (end 155.0543 71.25208) (width 0.2) (layer F.Cu) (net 4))
 (segment (start 153.551 71.997) (end 154.30938 71.997) (width 0.2) (layer F.Cu) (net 4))
 (segment (start 152.101 67.0467) (end 150.0324 67.0467) (width 0.2) (layer F.Cu) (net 2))
 (segment (start 150.0324 67.0467) (end 149.7159 66.7302) (width 0.2) (layer F.Cu) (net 2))
 (segment (start 143.9253 68.7885) (end 147.6576 68.7885) (width 0.2) (layer B.Cu) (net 2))
 (segment (start 147.6576 68.7885) (end 149.7159 66.7302) (width 0.2) (layer B.Cu) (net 2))
 (segment (start 152.101 68.147) (end 152.101 67.0467) (width 0.2) (layer F.Cu) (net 2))
 (segment (start 140.3073 68.83) (end 140.3488 68.7885) (width 0.2) (layer F.Cu) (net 2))
 (segment (start 140.3488 68.7885) (end 143.9253 68.7885) (width 0.2) (layer F.Cu) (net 2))
 (segment (start 139.507 68.83) (end 140.3073 68.83) (width 0.2) (layer F.Cu) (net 2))
 (via (at 143.9253 68.7885) (size 0.8) (layers F.Cu B.Cu) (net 2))
 (via (at 149.7159 66.7302) (size 0.8) (layers F.Cu B.Cu) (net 2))
 (segment (start 142.838725 65.68) (end 142.830731 65.694827) (width 0.2) (layer F.Cu) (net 2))
 (segment (start 143.9253 68.7885) (end 142.403701 67.266901) (width 0.2) (layer F.Cu) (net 2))
 (segment (start 142.4604 65.68) (end 142.838725 65.68) (width 0.2) (layer F.Cu) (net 2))
 (segment (start 142.403701 65.736699) (end 142.4604 65.68) (width 0.2) (layer F.Cu) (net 2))
 (segment (start 142.403701 67.266901) (end 142.403701 65.736699) (width 0.2) (layer F.Cu) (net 2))
 (segment (start 153.551 70.397) (end 154.6513 70.397) (width 0.2) (layer F.Cu) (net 6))
 (segment (start 154.6513 64.106118) (end 153.363681 62.818499) (width 0.2) (layer F.Cu) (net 6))
 (segment (start 154.6513 70.397) (end 154.6513 64.106118) (width 0.2) (layer F.Cu) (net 6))
 (segment (start 140.3073 65.3098) (end 144.7197 60.8974) (width 0.2) (layer B.Cu) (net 6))
 (segment (start 151.134761 60.8974) (end 152.336898 62.099537) (width 0.2) (layer B.Cu) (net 6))
 (segment (start 139.507 68.83) (end 140.3073 68.83) (width 0.2) (layer B.Cu) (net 6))
 (segment (start 144.7197 60.8974) (end 151.134761 60.8974) (width 0.2) (layer B.Cu) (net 6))
 (segment (start 140.3073 68.83) (end 140.3073 65.3098) (width 0.2) (layer B.Cu) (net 6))
 (segment (start 152.4507 69.597) (end 152.1238 69.597) (width 0.2) (layer F.Cu) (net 5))
 (segment (start 143.6478 71.195) (end 150.5258 71.195) (width 0.2) (layer B.Cu) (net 5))
 (segment (start 150.5258 71.195) (end 152.1238 69.597) (width 0.2) (layer B.Cu) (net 5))
 (segment (start 153.551 69.597) (end 152.4507 69.597) (width 0.2) (layer F.Cu) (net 5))
 (segment (start 140.3073 71.37) (end 140.4823 71.195) (width 0.2) (layer F.Cu) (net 5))
 (segment (start 140.4823 71.195) (end 143.6478 71.195) (width 0.2) (layer F.Cu) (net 5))
 (segment (start 139.507 71.37) (end 140.3073 71.37) (width 0.2) (layer F.Cu) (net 5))
 (via (at 143.6478 71.195) (size 0.8) (layers F.Cu B.Cu) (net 5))
 (via (at 152.1238 69.597) (size 0.8) (layers F.Cu B.Cu) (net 5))
 (segment (start 151.810256 65.170463) (end 151.731581 65.149382) (width 0.2) (layer F.Cu) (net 5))
 (segment (start 153.551 69.597) (end 153.551 66.911207) (width 0.2) (layer F.Cu) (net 5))
 (segment (start 153.551 66.911207) (end 151.810256 65.170463) (width 0.2) (layer F.Cu) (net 5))
 (segment (start 143.6384 72.797) (end 143.6384 72.2309) (width 0.2) (layer B.Cu) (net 9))
 (segment (start 143.6384 72.2309) (end 141.7037 70.2962) (width 0.2) (layer B.Cu) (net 9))
 (segment (start 141.7037 70.2962) (end 141.7037 66.0727) (width 0.2) (layer B.Cu) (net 9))
 (segment (start 140.5246 65.2107) (end 140.5246 66.0727) (width 0.2) (layer F.Cu) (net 9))
 (segment (start 140.5246 66.0727) (end 141.7037 66.0727) (width 0.2) (layer F.Cu) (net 9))
 (segment (start 140.3073 66.29) (end 140.5246 66.0727) (width 0.2) (layer F.Cu) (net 9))
 (segment (start 139.507 66.29) (end 140.3073 66.29) (width 0.2) (layer F.Cu) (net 9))
 (segment (start 145.051 72.797) (end 143.6384 72.797) (width 0.2) (layer F.Cu) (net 9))
 (via (at 143.6384 72.797) (size 0.8) (layers F.Cu B.Cu) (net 9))
 (via (at 141.7037 66.0727) (size 0.8) (layers F.Cu B.Cu) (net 9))
 (segment (start 140.5246 65.2107) (end 139.6835 65.2107) (width 0.2) (layer F.Cu) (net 9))
 (segment (start 139.553719 65.080919) (end 139.553719 63.374501) (width 0.2) (layer F.Cu) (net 9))
 (segment (start 139.6835 65.2107) (end 139.553719 65.080919) (width 0.2) (layer F.Cu) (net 9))
 (segment (start 142.034 62.6136) (end 141.81308 62.83452) (width 0.2) (layer F.Cu) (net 9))
 (segment (start 142.509 62.6136) (end 142.034 62.6136) (width 0.2) (layer F.Cu) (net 9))
 (segment (start 141.81308 62.83452) (end 140.9827 62.83452) (width 0.2) (layer F.Cu) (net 9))
 (segment (start 136.348 66.29) (end 138.207 66.29) (width 0.2) (layer B.Cu) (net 7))
 (segment (start 133.808 66.29) (end 134.9583 66.29) (width 0.2) (layer F.Cu) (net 8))
 (segment (start 134.9583 66.29) (end 134.9583 66.5776) (width 0.2) (layer F.Cu) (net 8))
 (segment (start 134.9583 66.5776) (end 135.8354 67.4547) (width 0.2) (layer F.Cu) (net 8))
 (segment (start 135.8354 67.4547) (end 137.0423 67.4547) (width 0.2) (layer F.Cu) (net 8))
 (segment (start 137.0423 67.4547) (end 138.207 66.29) (width 0.2) (layer F.Cu) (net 8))
 (segment (start 136.348 68.83) (end 138.207 68.83) (width 0.2) (layer B.Cu) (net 10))
 (segment (start 133.808 68.83) (end 134.9583 68.83) (width 0.2) (layer F.Cu) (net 11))
 (segment (start 138.207 68.83) (end 137.0164 70.0206) (width 0.2) (layer F.Cu) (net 11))
 (segment (start 137.0164 70.0206) (end 135.9105 70.0206) (width 0.2) (layer F.Cu) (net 11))
 (segment (start 135.9105 70.0206) (end 134.9583 69.0684) (width 0.2) (layer F.Cu) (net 11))
 (segment (start 134.9583 69.0684) (end 134.9583 68.83) (width 0.2) (layer F.Cu) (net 11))
 (segment (start 139.507 71.7508) (end 139.507 71.37) (width 0.2) (layer B.Cu) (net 3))
 (segment (start 140.207 71.37) (end 140.7479 70.8291) (width 0.2) (layer B.Cu) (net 3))
 (segment (start 140.7479 70.8291) (end 140.7479 70.3197) (width 0.2) (layer B.Cu) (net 3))
 (segment (start 139.507 71.37) (end 140.207 71.37) (width 0.2) (layer B.Cu) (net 3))
 (segment (start 136.348 71.37) (end 138.207 71.37) (width 0.2) (layer B.Cu) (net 12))
 (segment (start 133.808 71.37) (end 134.9583 71.37) (width 0.2) (layer F.Cu) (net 13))
 (segment (start 134.9583 71.37) (end 134.9583 71.6576) (width 0.2) (layer F.Cu) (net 13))
 (segment (start 134.9583 71.6576) (end 135.8385 72.5378) (width 0.2) (layer F.Cu) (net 13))
 (segment (start 135.8385 72.5378) (end 137.0392 72.5378) (width 0.2) (layer F.Cu) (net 13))
 (segment (start 137.0392 72.5378) (end 138.207 71.37) (width 0.2) (layer F.Cu) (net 13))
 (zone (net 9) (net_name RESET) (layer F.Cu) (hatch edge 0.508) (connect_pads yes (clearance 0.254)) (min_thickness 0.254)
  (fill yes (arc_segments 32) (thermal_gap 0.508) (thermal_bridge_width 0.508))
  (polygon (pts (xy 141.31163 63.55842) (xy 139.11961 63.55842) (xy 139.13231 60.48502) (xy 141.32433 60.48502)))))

